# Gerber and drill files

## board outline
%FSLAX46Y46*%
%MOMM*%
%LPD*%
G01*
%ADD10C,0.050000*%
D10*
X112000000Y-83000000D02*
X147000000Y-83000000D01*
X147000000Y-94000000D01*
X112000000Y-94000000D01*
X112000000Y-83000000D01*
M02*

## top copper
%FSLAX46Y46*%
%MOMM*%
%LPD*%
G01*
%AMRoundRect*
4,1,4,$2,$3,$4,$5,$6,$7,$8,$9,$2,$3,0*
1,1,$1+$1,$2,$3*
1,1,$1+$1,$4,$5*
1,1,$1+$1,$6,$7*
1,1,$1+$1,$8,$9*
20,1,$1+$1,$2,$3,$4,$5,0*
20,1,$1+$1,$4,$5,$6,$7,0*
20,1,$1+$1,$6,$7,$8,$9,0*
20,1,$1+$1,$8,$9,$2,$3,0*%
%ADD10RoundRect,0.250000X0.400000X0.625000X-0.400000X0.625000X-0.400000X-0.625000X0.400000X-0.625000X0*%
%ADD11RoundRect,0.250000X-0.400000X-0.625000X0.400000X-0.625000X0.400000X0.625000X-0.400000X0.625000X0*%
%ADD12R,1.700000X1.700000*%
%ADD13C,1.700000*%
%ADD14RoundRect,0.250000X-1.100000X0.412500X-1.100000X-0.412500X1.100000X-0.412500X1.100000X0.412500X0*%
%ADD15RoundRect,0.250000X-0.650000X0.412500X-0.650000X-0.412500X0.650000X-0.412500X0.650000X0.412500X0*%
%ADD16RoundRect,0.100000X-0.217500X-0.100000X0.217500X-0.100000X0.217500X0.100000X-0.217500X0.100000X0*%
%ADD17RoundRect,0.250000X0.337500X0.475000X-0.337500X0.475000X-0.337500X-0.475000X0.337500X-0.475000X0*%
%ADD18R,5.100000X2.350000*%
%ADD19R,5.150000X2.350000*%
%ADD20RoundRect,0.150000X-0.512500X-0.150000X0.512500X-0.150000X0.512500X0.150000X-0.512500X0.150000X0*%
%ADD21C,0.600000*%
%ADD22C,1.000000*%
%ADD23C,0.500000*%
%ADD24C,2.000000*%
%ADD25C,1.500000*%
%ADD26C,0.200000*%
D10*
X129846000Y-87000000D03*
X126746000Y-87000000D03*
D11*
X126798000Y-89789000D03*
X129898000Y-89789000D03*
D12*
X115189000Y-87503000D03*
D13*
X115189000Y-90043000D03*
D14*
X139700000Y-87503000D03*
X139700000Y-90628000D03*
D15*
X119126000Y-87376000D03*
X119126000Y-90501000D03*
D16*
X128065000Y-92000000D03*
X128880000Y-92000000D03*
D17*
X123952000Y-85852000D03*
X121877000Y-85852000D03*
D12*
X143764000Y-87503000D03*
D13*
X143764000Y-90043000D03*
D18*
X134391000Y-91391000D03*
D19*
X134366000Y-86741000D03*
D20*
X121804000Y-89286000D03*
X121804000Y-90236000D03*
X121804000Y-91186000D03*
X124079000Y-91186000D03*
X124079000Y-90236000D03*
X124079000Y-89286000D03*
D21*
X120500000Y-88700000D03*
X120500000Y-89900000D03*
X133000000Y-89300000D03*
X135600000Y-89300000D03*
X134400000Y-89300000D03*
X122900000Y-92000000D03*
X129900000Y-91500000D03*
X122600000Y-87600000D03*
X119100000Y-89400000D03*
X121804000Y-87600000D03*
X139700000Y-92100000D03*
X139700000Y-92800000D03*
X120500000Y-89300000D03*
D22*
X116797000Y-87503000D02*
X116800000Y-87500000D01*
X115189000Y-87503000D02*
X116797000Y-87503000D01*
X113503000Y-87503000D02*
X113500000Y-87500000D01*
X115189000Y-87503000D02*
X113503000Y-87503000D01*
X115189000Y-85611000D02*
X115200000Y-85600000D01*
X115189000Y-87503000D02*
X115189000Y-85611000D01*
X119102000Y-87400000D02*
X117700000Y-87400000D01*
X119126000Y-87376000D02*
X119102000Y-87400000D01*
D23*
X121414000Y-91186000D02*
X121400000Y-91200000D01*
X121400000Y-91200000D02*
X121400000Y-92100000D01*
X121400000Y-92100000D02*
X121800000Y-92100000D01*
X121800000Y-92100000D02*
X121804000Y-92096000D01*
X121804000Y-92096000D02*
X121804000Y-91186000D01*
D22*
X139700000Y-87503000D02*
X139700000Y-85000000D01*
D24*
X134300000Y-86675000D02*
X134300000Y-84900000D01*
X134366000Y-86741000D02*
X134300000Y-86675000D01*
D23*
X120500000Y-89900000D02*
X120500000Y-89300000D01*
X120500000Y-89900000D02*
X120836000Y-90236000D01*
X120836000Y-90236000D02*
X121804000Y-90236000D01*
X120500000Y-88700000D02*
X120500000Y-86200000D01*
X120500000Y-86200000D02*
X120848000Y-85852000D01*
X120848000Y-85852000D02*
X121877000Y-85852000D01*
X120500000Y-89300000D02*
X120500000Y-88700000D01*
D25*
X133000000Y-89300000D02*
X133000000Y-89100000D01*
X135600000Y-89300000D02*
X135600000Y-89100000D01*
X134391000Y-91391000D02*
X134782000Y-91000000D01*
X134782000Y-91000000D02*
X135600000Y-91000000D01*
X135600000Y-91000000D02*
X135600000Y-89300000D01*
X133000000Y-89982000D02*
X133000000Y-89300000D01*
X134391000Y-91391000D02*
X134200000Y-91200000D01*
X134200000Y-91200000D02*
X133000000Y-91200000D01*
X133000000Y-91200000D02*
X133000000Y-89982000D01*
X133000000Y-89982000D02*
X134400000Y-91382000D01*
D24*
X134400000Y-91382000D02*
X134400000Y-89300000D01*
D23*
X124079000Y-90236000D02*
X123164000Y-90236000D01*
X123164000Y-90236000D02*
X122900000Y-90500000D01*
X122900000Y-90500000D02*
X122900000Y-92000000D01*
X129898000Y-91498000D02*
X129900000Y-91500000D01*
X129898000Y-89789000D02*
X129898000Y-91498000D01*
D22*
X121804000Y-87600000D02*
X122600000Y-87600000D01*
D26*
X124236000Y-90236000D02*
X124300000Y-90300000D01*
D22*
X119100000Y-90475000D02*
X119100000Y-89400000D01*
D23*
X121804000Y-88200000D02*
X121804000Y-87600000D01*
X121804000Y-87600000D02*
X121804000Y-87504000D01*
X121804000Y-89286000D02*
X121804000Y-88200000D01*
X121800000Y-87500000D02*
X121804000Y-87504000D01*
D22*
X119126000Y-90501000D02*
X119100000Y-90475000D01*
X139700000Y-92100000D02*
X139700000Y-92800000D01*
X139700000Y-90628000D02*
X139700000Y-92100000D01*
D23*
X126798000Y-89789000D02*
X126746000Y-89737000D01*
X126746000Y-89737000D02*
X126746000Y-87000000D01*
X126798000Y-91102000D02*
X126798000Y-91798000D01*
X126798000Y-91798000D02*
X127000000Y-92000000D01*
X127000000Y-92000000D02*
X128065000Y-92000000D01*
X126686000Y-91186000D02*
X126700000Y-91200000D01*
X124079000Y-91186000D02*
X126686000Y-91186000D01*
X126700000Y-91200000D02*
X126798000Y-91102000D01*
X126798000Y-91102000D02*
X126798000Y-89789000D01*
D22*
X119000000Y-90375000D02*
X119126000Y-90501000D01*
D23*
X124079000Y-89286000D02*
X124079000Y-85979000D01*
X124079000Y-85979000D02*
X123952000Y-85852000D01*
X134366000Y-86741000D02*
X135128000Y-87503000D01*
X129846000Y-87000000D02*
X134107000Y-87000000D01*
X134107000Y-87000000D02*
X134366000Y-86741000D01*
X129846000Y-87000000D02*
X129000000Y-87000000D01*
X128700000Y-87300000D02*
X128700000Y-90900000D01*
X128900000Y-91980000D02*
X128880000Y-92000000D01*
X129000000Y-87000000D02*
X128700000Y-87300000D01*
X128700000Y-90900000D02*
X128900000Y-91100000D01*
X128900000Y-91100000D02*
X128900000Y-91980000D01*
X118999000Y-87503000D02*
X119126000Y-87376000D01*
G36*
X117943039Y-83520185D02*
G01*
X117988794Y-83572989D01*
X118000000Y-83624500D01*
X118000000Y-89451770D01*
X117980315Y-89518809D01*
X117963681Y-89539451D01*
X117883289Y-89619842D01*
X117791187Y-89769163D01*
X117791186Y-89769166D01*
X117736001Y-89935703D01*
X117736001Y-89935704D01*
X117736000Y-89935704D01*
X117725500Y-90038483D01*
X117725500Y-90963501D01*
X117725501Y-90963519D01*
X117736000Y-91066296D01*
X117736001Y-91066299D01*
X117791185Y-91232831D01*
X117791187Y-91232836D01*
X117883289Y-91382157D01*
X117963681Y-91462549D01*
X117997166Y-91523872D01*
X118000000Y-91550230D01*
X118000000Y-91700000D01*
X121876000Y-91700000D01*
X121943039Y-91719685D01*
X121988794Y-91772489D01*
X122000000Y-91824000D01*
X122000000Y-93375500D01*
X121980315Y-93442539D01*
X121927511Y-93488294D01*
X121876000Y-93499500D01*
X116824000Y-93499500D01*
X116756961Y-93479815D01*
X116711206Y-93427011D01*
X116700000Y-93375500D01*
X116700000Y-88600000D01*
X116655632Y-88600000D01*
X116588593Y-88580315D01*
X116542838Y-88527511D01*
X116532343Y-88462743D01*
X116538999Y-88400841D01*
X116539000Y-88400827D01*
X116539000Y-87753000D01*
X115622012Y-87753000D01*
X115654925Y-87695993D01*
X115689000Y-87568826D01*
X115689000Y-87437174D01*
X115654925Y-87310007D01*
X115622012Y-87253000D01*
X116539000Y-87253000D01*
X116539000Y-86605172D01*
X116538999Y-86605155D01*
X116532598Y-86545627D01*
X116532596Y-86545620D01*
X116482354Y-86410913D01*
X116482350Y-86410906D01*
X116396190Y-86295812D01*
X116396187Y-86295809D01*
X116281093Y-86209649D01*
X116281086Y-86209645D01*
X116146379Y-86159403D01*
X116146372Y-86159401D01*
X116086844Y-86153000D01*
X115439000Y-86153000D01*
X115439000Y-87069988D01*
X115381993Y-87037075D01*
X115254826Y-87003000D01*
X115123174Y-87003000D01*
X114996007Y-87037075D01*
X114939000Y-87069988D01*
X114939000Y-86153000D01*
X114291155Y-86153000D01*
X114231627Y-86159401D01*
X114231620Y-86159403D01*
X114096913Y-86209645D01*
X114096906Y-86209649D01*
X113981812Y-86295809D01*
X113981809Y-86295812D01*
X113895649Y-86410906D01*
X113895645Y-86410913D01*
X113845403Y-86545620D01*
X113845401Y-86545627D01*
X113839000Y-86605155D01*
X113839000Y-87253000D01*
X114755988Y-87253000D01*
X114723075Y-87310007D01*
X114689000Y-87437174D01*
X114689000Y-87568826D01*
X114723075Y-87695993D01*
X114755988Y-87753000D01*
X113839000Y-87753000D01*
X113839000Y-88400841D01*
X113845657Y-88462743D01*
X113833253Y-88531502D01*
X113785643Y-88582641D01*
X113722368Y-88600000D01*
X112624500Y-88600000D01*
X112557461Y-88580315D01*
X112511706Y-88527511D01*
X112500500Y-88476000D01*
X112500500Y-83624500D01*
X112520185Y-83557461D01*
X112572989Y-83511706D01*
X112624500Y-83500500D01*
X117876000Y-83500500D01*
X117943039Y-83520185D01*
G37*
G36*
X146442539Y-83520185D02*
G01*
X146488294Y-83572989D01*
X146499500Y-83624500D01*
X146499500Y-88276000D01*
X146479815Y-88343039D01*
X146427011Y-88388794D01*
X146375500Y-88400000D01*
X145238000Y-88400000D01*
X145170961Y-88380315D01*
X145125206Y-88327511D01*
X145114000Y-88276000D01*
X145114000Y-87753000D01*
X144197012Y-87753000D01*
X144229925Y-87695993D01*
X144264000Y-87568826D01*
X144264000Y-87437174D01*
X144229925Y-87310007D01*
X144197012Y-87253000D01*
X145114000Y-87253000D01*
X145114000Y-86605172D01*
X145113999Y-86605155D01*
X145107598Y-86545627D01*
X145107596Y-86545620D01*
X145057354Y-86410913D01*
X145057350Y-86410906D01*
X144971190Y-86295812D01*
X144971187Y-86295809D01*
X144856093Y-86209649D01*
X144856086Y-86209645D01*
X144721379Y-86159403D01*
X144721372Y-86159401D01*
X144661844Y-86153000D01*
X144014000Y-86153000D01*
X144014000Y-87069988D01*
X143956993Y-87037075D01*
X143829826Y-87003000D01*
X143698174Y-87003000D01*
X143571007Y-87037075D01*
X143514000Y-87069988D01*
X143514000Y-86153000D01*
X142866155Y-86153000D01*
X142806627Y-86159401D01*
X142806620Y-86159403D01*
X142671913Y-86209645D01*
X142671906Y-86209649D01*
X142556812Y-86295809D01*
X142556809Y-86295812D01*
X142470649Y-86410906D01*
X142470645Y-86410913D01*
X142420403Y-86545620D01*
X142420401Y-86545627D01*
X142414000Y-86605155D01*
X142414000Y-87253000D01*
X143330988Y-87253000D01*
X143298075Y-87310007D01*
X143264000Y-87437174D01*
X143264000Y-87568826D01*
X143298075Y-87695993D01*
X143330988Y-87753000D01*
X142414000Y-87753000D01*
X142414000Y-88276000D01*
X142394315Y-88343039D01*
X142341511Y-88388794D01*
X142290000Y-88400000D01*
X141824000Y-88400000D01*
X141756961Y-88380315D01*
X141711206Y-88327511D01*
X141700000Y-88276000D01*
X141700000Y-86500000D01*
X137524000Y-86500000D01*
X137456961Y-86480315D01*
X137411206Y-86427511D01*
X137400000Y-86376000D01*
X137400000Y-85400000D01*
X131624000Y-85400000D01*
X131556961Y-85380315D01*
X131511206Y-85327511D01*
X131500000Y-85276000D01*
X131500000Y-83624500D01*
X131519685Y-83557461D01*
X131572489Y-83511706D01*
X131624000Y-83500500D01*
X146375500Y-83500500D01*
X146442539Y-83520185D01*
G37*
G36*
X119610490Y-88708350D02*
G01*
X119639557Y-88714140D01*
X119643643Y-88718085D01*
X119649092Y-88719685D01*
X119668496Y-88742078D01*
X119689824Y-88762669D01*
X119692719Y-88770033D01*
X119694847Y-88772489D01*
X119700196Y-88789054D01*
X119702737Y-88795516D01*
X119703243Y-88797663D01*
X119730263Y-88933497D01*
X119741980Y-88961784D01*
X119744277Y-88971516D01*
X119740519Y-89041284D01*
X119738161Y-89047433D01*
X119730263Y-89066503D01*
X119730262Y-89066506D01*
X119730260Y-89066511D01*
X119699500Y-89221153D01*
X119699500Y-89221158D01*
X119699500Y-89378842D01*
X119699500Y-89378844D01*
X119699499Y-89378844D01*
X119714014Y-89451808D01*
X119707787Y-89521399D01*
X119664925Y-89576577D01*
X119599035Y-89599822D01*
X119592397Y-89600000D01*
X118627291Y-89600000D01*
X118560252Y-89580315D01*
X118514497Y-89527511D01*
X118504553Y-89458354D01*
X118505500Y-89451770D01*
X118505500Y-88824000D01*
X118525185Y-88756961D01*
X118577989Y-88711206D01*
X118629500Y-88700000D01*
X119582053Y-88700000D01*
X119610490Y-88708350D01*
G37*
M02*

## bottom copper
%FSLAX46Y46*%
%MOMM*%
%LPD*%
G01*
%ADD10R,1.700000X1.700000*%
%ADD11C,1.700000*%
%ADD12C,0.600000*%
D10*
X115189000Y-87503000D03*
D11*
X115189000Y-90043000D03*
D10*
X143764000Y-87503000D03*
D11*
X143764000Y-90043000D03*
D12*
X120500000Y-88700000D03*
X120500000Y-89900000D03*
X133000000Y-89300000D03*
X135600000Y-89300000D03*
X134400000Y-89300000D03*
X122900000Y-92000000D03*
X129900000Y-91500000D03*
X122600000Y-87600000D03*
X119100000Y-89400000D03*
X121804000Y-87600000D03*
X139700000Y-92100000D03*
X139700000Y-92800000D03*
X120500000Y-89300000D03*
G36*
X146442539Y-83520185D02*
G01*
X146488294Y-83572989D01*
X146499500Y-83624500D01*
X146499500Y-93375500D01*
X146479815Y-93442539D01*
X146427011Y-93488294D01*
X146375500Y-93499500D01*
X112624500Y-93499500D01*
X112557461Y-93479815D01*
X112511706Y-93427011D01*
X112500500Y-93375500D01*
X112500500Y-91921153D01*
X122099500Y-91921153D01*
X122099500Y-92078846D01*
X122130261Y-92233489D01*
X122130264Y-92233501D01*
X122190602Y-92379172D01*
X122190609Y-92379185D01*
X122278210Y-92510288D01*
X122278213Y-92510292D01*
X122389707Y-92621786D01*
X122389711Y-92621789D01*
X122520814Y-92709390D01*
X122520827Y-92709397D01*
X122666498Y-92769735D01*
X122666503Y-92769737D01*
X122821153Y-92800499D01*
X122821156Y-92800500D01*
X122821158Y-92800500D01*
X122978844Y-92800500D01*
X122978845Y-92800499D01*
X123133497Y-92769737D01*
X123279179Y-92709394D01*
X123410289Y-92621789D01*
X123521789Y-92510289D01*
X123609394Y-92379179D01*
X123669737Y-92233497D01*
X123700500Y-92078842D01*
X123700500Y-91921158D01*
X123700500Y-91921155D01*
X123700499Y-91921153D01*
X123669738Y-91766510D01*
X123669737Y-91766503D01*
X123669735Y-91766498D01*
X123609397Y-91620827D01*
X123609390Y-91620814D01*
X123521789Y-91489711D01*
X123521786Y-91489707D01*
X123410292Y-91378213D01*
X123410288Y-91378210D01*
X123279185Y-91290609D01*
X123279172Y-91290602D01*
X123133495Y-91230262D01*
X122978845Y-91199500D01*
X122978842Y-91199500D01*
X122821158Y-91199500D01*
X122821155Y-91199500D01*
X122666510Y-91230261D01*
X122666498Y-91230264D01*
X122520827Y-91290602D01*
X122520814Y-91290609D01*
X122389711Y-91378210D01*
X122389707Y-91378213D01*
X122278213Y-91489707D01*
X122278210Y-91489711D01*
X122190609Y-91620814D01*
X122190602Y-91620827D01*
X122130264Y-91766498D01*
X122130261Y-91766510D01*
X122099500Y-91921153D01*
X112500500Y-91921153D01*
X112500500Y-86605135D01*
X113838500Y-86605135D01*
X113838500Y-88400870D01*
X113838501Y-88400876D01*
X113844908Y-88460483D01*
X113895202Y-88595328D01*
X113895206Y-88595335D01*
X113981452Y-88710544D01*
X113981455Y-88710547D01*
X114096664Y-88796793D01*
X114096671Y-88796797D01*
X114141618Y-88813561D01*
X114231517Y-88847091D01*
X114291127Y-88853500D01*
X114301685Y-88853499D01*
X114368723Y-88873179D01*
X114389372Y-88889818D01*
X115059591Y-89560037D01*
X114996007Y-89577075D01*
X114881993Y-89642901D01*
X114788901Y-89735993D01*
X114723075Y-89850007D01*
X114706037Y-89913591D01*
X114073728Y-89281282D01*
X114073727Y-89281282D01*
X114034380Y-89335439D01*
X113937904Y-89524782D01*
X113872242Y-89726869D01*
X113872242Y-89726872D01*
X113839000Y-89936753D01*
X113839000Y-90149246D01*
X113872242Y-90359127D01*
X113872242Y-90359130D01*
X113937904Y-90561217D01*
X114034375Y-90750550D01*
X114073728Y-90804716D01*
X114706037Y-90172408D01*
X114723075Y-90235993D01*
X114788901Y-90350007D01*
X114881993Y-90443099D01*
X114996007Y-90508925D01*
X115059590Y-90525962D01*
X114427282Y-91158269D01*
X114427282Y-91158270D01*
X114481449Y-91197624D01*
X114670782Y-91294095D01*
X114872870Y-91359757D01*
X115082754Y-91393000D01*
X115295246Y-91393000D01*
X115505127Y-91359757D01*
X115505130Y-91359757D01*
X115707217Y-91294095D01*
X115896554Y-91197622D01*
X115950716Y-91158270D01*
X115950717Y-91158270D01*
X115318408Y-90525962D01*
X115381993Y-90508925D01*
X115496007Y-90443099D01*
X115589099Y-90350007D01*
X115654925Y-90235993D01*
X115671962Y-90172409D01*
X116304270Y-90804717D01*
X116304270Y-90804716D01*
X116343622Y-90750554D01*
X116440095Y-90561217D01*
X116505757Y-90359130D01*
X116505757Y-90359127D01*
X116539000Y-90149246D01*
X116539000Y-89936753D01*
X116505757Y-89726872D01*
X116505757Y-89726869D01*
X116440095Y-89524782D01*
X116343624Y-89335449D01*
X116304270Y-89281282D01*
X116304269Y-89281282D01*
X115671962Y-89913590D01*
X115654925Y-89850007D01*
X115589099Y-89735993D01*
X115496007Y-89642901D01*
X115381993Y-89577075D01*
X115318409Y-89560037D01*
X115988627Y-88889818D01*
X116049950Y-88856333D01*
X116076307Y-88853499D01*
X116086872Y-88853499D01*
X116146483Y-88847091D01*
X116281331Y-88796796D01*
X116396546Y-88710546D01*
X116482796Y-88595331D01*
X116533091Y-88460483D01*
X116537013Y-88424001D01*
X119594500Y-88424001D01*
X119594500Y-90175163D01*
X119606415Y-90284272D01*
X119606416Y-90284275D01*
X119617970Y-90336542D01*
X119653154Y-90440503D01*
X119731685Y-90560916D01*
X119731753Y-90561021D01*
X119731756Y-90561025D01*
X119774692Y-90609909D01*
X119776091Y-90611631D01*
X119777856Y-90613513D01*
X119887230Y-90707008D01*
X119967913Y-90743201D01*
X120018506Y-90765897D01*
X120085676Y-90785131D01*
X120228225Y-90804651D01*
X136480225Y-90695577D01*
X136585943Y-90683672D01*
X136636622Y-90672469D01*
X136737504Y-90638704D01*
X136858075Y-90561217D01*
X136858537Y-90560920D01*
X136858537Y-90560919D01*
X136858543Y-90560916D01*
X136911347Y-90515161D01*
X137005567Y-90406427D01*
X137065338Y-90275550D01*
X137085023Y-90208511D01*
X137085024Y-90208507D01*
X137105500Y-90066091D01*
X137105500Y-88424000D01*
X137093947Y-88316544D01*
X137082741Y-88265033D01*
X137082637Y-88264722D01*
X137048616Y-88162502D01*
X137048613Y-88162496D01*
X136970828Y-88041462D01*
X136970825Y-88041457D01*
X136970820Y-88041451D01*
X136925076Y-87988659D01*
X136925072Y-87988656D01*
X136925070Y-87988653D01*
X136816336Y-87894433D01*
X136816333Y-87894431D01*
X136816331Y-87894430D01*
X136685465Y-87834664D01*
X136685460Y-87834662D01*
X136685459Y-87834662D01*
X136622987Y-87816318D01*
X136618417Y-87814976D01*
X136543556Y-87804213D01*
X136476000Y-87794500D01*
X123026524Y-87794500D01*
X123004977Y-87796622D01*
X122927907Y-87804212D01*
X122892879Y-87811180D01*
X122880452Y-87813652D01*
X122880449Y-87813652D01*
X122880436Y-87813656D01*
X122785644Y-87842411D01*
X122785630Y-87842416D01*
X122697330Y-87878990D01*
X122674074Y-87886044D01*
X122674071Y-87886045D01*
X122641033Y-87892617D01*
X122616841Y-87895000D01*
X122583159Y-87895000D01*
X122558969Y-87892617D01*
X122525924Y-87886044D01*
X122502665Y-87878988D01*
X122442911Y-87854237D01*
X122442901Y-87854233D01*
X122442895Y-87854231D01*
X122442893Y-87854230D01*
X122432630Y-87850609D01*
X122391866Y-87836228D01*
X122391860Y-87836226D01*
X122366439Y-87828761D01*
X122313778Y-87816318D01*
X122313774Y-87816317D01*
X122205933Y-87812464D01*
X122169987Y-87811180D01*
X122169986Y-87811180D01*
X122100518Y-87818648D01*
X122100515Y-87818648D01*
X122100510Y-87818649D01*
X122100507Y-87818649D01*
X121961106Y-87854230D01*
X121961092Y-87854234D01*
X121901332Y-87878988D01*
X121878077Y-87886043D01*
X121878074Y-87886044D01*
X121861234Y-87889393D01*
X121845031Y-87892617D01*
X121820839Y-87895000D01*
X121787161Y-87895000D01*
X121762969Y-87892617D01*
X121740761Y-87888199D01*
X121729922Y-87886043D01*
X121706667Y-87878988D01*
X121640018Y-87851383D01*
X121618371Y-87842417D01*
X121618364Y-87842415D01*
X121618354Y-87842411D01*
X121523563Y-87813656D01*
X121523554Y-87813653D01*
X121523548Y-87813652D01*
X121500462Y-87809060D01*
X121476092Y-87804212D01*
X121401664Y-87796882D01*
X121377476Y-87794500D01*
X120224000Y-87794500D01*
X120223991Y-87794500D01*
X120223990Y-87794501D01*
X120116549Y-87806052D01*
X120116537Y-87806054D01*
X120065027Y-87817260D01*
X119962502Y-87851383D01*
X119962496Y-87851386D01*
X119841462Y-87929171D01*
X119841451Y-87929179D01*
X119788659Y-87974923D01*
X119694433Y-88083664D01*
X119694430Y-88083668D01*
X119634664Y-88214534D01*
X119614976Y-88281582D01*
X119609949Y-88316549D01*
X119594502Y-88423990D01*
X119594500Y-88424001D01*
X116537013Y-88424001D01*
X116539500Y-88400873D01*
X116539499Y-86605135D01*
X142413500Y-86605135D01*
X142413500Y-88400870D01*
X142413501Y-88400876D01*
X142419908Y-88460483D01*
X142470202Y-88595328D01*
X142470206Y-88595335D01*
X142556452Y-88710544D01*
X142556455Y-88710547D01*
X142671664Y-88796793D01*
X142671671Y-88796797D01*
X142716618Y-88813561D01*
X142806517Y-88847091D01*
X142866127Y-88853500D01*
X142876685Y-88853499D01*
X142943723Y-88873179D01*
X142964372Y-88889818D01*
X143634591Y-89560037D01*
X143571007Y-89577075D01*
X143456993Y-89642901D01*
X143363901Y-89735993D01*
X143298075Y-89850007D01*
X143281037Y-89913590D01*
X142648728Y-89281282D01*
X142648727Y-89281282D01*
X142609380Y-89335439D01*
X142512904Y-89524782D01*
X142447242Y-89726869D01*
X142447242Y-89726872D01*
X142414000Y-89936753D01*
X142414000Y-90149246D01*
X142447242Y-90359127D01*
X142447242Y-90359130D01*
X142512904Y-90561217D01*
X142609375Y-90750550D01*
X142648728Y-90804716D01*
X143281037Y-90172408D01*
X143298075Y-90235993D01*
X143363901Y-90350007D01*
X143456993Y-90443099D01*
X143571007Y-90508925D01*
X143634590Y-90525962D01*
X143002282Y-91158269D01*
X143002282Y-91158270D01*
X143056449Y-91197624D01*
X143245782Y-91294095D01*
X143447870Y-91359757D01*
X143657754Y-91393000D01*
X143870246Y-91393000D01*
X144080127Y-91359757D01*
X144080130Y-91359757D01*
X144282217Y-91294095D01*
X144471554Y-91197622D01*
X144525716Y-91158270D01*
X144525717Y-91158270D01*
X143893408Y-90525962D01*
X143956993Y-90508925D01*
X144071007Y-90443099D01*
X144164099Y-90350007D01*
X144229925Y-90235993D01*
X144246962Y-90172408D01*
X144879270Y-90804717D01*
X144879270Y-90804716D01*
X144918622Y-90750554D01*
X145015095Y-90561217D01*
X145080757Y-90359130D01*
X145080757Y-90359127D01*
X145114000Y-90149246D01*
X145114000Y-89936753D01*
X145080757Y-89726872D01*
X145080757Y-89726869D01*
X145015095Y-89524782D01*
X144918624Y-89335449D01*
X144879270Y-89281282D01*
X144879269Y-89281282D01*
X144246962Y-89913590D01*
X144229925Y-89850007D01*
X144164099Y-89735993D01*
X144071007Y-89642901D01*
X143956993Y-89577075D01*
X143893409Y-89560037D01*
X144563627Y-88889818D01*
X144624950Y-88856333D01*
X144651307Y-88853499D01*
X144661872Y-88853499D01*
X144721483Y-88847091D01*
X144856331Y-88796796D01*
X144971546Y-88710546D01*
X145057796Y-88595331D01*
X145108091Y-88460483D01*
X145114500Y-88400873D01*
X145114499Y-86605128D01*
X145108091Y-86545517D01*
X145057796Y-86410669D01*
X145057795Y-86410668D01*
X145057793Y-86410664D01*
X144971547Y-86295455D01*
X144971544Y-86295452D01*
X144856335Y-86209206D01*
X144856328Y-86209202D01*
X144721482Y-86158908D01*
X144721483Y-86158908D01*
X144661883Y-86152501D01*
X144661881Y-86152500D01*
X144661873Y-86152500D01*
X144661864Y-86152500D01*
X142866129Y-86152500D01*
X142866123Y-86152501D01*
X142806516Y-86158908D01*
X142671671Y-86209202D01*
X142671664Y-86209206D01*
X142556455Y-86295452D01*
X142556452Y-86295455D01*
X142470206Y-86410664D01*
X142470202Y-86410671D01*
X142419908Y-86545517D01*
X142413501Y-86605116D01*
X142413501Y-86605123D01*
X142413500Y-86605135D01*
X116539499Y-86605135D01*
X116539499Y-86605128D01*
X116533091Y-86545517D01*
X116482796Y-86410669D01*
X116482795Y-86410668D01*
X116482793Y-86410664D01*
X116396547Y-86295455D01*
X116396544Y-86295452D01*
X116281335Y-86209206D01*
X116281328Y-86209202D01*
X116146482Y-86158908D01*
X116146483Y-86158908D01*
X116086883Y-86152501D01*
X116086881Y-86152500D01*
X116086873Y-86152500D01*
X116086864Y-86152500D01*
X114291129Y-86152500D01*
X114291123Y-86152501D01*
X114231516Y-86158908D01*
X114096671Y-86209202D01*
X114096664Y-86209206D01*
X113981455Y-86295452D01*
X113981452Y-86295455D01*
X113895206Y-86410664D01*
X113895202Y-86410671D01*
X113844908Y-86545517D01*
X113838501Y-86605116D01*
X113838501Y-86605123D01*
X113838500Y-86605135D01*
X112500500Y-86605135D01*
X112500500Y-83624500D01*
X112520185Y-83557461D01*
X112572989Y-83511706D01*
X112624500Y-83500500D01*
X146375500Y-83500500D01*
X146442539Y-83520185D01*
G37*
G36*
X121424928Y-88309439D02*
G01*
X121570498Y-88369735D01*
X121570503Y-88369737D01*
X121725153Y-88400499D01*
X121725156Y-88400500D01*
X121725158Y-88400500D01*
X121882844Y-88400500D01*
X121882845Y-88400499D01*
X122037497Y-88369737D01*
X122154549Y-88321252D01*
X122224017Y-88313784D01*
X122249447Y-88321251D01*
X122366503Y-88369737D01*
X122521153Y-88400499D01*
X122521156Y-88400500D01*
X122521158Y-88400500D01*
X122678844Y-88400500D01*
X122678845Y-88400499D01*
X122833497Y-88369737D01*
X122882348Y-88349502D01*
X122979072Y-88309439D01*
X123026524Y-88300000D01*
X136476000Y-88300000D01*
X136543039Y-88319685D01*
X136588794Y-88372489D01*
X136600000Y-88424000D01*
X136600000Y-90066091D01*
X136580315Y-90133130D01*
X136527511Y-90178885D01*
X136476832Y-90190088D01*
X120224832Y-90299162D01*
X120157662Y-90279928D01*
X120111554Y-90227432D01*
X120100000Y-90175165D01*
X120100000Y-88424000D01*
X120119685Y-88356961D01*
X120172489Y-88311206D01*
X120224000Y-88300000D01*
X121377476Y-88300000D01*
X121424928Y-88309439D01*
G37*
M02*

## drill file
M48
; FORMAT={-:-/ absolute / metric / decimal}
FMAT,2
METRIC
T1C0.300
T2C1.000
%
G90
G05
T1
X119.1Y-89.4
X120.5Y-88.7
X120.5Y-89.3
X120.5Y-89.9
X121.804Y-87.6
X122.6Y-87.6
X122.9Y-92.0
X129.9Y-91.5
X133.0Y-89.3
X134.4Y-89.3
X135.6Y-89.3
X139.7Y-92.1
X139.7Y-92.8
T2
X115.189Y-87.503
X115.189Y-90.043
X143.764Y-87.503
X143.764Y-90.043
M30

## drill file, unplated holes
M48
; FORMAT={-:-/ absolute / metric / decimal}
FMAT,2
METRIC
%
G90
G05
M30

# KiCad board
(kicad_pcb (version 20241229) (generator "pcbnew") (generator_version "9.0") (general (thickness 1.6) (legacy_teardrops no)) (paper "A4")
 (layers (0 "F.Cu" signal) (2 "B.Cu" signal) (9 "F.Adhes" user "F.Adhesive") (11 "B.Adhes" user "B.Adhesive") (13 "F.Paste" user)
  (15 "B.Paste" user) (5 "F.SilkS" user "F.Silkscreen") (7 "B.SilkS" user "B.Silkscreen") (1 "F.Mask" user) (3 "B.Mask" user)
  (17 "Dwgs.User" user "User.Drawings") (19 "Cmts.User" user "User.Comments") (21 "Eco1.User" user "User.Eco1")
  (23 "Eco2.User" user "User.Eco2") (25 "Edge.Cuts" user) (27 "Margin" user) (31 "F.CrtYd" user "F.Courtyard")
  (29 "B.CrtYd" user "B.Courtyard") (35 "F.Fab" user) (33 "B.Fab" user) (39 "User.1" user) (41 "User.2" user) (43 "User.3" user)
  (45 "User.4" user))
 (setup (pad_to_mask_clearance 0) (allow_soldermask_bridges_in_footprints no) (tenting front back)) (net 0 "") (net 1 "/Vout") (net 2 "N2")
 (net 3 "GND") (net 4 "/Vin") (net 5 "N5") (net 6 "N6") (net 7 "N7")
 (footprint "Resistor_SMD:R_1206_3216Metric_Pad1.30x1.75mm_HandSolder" (layer "F.Cu") (at 128.296 87 180)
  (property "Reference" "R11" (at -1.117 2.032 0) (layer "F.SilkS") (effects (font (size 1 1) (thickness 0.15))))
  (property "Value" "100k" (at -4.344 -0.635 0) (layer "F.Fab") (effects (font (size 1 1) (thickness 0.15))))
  (pad "1" smd roundrect (at -1.55 0 180) (size 1.3 1.75) (layers "F.Cu" "F.Mask" "F.Paste") (roundrect_rratio 0.192308) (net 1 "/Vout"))
  (pad "2" smd roundrect (at 1.55 0 180) (size 1.3 1.75) (layers "F.Cu" "F.Mask" "F.Paste") (roundrect_rratio 0.192308) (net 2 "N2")))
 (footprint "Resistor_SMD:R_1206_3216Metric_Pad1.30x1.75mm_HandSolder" (layer "F.Cu") (at 128.348 89.789)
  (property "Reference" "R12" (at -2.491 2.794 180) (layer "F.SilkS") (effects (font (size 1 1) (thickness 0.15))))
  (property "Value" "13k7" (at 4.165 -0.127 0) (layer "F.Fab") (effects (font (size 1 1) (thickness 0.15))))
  (pad "1" smd roundrect (at -1.55 0) (size 1.3 1.75) (layers "F.Cu" "F.Mask" "F.Paste") (roundrect_rratio 0.192308) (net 2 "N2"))
  (pad "2" smd roundrect (at 1.55 0) (size 1.3 1.75) (layers "F.Cu" "F.Mask" "F.Paste") (roundrect_rratio 0.192308) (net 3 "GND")))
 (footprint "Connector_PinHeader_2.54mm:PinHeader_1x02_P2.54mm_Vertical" (layer "F.Cu") (at 115.189 87.503)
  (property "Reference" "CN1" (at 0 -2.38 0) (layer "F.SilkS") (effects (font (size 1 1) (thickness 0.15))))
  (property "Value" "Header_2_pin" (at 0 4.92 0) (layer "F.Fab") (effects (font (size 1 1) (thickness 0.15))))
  (pad "1" thru_hole rect (at 0 0) (size 1.7 1.7) (drill 1) (layers "*.Cu" "*.Mask") (remove_unused_layers no) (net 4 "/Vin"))
  (pad "2" thru_hole circle (at 0 2.54) (size 1.7 1.7) (drill 1) (layers "*.Cu" "*.Mask") (remove_unused_layers no) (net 3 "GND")))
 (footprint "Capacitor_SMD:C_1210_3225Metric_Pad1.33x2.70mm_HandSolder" (layer "F.Cu") (at 139.7 89.0655 -90)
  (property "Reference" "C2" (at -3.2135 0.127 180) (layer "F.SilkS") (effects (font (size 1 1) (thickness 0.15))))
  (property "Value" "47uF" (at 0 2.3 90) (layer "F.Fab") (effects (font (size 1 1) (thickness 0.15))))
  (pad "1" smd roundrect (at -1.5625 0 270) (size 1.325 2.7) (layers "F.Cu" "F.Mask" "F.Paste") (roundrect_rratio 0.188679) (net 1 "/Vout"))
  (pad "2" smd roundrect (at 1.5625 0 270) (size 1.325 2.7) (layers "F.Cu" "F.Mask" "F.Paste") (roundrect_rratio 0.188679) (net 3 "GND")))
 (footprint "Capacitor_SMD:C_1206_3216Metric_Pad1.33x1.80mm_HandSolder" (layer "F.Cu") (at 119.126 88.9385 -90)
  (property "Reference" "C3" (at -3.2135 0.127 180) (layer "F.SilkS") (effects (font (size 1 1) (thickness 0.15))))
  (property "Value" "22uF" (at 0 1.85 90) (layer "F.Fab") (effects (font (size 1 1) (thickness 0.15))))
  (pad "1" smd roundrect (at -1.5625 0 270) (size 1.325 1.8) (layers "F.Cu" "F.Mask" "F.Paste") (roundrect_rratio 0.188679) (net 4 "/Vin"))
  (pad "2" smd roundrect (at 1.5625 0 270) (size 1.325 1.8) (layers "F.Cu" "F.Mask" "F.Paste") (roundrect_rratio 0.188679) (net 3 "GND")))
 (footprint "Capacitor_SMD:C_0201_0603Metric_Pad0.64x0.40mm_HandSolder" (layer "F.Cu") (at 128.4725 92)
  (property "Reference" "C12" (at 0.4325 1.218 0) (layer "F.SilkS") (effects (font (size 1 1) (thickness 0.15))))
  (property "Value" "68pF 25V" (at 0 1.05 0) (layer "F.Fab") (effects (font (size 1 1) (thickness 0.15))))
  (pad "" smd roundrect (at -0.4325 0) (size 0.458 0.36) (layers "F.Paste") (roundrect_rratio 0.25))
  (pad "" smd roundrect (at 0.4325 0) (size 0.458 0.36) (layers "F.Paste") (roundrect_rratio 0.25))
  (pad "1" smd roundrect (at -0.4075 0) (size 0.635 0.4) (layers "F.Cu" "F.Mask") (roundrect_rratio 0.25) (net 2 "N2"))
  (pad "2" smd roundrect (at 0.4075 0) (size 0.635 0.4) (layers "F.Cu" "F.Mask") (roundrect_rratio 0.25) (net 1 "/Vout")))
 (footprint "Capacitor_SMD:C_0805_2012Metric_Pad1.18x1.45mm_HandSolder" (layer "F.Cu") (at 122.9145 85.852 180)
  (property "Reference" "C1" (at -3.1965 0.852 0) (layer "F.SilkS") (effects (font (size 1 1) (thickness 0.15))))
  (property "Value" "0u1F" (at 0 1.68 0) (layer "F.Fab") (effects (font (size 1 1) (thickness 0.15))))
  (pad "1" smd roundrect (at -1.0375 0 180) (size 1.175 1.45) (layers "F.Cu" "F.Mask" "F.Paste") (roundrect_rratio 0.212766) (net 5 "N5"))
  (pad "2" smd roundrect (at 1.0375 0 180) (size 1.175 1.45) (layers "F.Cu" "F.Mask" "F.Paste") (roundrect_rratio 0.212766) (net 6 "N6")))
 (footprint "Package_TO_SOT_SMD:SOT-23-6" (layer "F.Cu") (at 122.9415 90.236)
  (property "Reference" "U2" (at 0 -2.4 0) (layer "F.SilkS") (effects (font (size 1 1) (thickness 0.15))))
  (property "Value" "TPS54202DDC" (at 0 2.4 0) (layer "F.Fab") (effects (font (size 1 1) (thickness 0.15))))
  (pad "1" smd roundrect (at -1.1375 -0.95) (size 1.325 0.6) (layers "F.Cu" "F.Mask" "F.Paste") (roundrect_rratio 0.25) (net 3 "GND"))
  (pad "2" smd roundrect (at -1.1375 0) (size 1.325 0.6) (layers "F.Cu" "F.Mask" "F.Paste") (roundrect_rratio 0.25) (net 6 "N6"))
  (pad "3" smd roundrect (at -1.1375 0.95) (size 1.325 0.6) (layers "F.Cu" "F.Mask" "F.Paste") (roundrect_rratio 0.25) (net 4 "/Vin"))
  (pad "4" smd roundrect (at 1.1375 0.95) (size 1.325 0.6) (layers "F.Cu" "F.Mask" "F.Paste") (roundrect_rratio 0.25) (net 2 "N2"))
  (pad "5" smd roundrect (at 1.1375 0) (size 1.325 0.6) (layers "F.Cu" "F.Mask" "F.Paste") (roundrect_rratio 0.25) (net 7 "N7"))
  (pad "6" smd roundrect (at 1.1375 -0.95) (size 1.325 0.6) (layers "F.Cu" "F.Mask" "F.Paste") (roundrect_rratio 0.25) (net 5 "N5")))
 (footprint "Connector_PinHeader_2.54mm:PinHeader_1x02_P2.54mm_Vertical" (layer "F.Cu") (at 143.764 87.503)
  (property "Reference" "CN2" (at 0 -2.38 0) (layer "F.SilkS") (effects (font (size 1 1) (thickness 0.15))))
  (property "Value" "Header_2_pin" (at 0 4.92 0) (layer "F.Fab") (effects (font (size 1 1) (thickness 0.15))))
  (pad "1" thru_hole rect (at 0 0) (size 1.7 1.7) (drill 1) (layers "*.Cu" "*.Mask") (remove_unused_layers no) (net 1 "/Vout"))
  (pad "2" thru_hole circle (at 0 2.54) (size 1.7 1.7) (drill 1) (layers "*.Cu" "*.Mask") (remove_unused_layers no) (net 3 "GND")))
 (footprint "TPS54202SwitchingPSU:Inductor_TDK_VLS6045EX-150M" (layer "F.Cu") (at 134.391 89.066 90)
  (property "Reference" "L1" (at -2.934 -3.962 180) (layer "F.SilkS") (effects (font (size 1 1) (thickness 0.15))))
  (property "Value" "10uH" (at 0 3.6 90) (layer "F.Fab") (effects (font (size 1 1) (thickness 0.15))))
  (pad "1" smd rect (at -2.325 0 90) (size 2.35 5.1) (layers "F.Cu" "F.Mask" "F.Paste") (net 6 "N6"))
  (pad "2" smd rect (at 2.325 -0.025 90) (size 2.35 5.15) (layers "F.Cu" "F.Mask" "F.Paste") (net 1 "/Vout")))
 (gr_rect (start 112 83) (end 147 94) (stroke (width 0.05) (type default)) (fill no) (layer "Edge.Cuts"))
 (segment (start 120.5 89.9) (end 120.5 89.3) (width 0.5) (layer "F.Cu") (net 6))
 (segment (start 133 89.3) (end 133 89.1) (width 1.5) (layer "F.Cu") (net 6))
 (segment (start 133 89.982) (end 134.4 91.382) (width 1.5) (layer "F.Cu") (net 6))
 (segment (start 120.5 89.9) (end 120.836 90.236) (width 0.5) (layer "F.Cu") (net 6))
 (segment (start 134.391 91.391) (end 134.2 91.2) (width 1.5) (layer "F.Cu") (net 6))
 (segment (start 120.5 86.2) (end 120.848 85.852) (width 0.5) (layer "F.Cu") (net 6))
 (segment (start 120.5 88.7) (end 120.5 86.2) (width 0.5) (layer "F.Cu") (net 6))
 (segment (start 120.836 90.236) (end 121.804 90.236) (width 0.5) (layer "F.Cu") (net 6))
 (segment (start 134.4 91.382) (end 134.4 89.3) (width 2) (layer "F.Cu") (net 6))
 (segment (start 133 89.982) (end 133 89.3) (width 1.5) (layer "F.Cu") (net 6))
 (segment (start 120.848 85.852) (end 121.877 85.852) (width 0.5) (layer "F.Cu") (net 6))
 (segment (start 120.5 89.3) (end 120.5 88.7) (width 0.5) (layer "F.Cu") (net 6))
 (segment (start 135.6 91) (end 135.6 89.3) (width 1.5) (layer "F.Cu") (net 6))
 (segment (start 134.391 91.391) (end 134.782 91) (width 1.5) (layer "F.Cu") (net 6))
 (segment (start 135.6 89.3) (end 135.6 89.1) (width 1.5) (layer "F.Cu") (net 6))
 (segment (start 133 91.2) (end 133 89.982) (width 1.5) (layer "F.Cu") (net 6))
 (segment (start 134.2 91.2) (end 133 91.2) (width 1.5) (layer "F.Cu") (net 6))
 (segment (start 134.782 91) (end 135.6 91) (width 1.5) (layer "F.Cu") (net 6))
 (via (at 120.5 89.9) (size 0.6) (drill 0.3) (layers "F.Cu" "B.Cu") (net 6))
 (via (at 120.5 89.3) (size 0.6) (drill 0.3) (layers "F.Cu" "B.Cu") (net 6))
 (via (at 133 89.3) (size 0.6) (drill 0.3) (layers "F.Cu" "B.Cu") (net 6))
 (via (at 135.6 89.3) (size 0.6) (drill 0.3) (layers "F.Cu" "B.Cu") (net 6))
 (via (at 134.4 89.3) (size 0.6) (drill 0.3) (layers "F.Cu" "B.Cu") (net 6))
 (via (at 120.5 88.7) (size 0.6) (drill 0.3) (layers "F.Cu" "B.Cu") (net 6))
 (segment (start 124.079 89.286) (end 124.079 85.979) (width 0.5) (layer "F.Cu") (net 5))
 (segment (start 124.079 85.979) (end 123.952 85.852) (width 0.5) (layer "F.Cu") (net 5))
 (segment (start 134.366 86.741) (end 134.3 86.675) (width 2) (layer "F.Cu") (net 1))
 (segment (start 134.107 87) (end 134.366 86.741) (width 0.5) (layer "F.Cu") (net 1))
 (segment (start 128.9 91.98) (end 128.88 92) (width 0.5) (layer "F.Cu") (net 1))
 (segment (start 139.7 87.503) (end 139.7 85) (width 1) (layer "F.Cu") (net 1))
 (segment (start 134.366 86.741) (end 135.128 87.503) (width 0.5) (layer "F.Cu") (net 1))
 (segment (start 129.846 87) (end 134.107 87) (width 0.5) (layer "F.Cu") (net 1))
 (segment (start 129 87) (end 128.7 87.3) (width 0.5) (layer "F.Cu") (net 1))
 (segment (start 129.846 87) (end 129 87) (width 0.5) (layer "F.Cu") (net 1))
 (segment (start 128.7 90.9) (end 128.9 91.1) (width 0.5) (layer "F.Cu") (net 1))
 (segment (start 128.9 91.1) (end 128.9 91.98) (width 0.5) (layer "F.Cu") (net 1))
 (segment (start 128.7 87.3) (end 128.7 90.9) (width 0.5) (layer "F.Cu") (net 1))
 (segment (start 134.3 86.675) (end 134.3 84.9) (width 2) (layer "F.Cu") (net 1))
 (segment (start 139.7 90.628) (end 139.7 92.1) (width 1) (layer "F.Cu") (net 3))
 (segment (start 129.898 89.789) (end 129.898 91.498) (width 0.5) (layer "F.Cu") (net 3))
 (segment (start 121.804 87.6) (end 121.804 87.504) (width 0.5) (layer "F.Cu") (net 3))
 (segment (start 119.1 90.475) (end 119.1 89.4) (width 1) (layer "F.Cu") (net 3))
 (segment (start 121.804 87.6) (end 122.6 87.6) (width 1) (layer "F.Cu") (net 3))
 (segment (start 121.804 89.286) (end 121.804 88.2) (width 0.5) (layer "F.Cu") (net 3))
 (segment (start 119.126 90.501) (end 119.1 90.475) (width 1) (layer "F.Cu") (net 3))
 (segment (start 121.8 87.5) (end 121.804 87.504) (width 0.5) (layer "F.Cu") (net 3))
 (segment (start 121.804 88.2) (end 121.804 87.6) (width 0.5) (layer "F.Cu") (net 3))
 (segment (start 129.898 91.498) (end 129.9 91.5) (width 0.5) (layer "F.Cu") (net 3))
 (segment (start 119 90.375) (end 119.126 90.501) (width 1) (layer "F.Cu") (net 3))
 (segment (start 139.7 92.1) (end 139.7 92.8) (width 1) (layer "F.Cu") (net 3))
 (via (at 139.7 92.1) (size 0.6) (drill 0.3) (layers "F.Cu" "B.Cu") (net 3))
 (via (at 121.804 87.6) (size 0.6) (drill 0.3) (layers "F.Cu" "B.Cu") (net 3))
 (via (at 139.7 92.8) (size 0.6) (drill 0.3) (layers "F.Cu" "B.Cu") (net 3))
 (via (at 119.1 89.4) (size 0.6) (drill 0.3) (layers "F.Cu" "B.Cu") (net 3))
 (via (at 129.9 91.5) (size 0.6) (drill 0.3) (layers "F.Cu" "B.Cu") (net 3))
 (via (at 122.6 87.6) (size 0.6) (drill 0.3) (layers "F.Cu" "B.Cu") (free yes) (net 3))
 (segment (start 121.4 91.2) (end 121.4 92.1) (width 0.5) (layer "F.Cu") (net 4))
 (segment (start 121.804 92.096) (end 121.804 91.186) (width 0.5) (layer "F.Cu") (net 4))
 (segment (start 113.503 87.503) (end 113.5 87.5) (width 1) (layer "F.Cu") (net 4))
 (segment (start 121.8 92.1) (end 121.804 92.096) (width 0.5) (layer "F.Cu") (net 4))
 (segment (start 119.102 87.4) (end 117.7 87.4) (width 1) (layer "F.Cu") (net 4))
 (segment (start 115.189 87.503) (end 116.797 87.503) (width 1) (layer "F.Cu") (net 4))
 (segment (start 115.189 87.503) (end 115.189 85.611) (width 1) (layer "F.Cu") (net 4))
 (segment (start 121.414 91.186) (end 121.4 91.2) (width 0.5) (layer "F.Cu") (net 4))
 (segment (start 116.797 87.503) (end 116.8 87.5) (width 1) (layer "F.Cu") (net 4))
 (segment (start 115.189 85.611) (end 115.2 85.6) (width 1) (layer "F.Cu") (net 4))
 (segment (start 121.4 92.1) (end 121.8 92.1) (width 0.5) (layer "F.Cu") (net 4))
 (segment (start 119.126 87.376) (end 119.102 87.4) (width 1) (layer "F.Cu") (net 4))
 (segment (start 118.999 87.503) (end 119.126 87.376) (width 0.5) (layer "F.Cu") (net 4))
 (segment (start 115.189 87.503) (end 113.503 87.503) (width 1) (layer "F.Cu") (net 4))
 (segment (start 126.798 91.102) (end 126.798 91.798) (width 0.5) (layer "F.Cu") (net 2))
 (segment (start 124.079 91.186) (end 126.686 91.186) (width 0.5) (layer "F.Cu") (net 2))
 (segment (start 126.798 91.798) (end 127 92) (width 0.5) (layer "F.Cu") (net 2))
 (segment (start 127 92) (end 128.065 92) (width 0.5) (layer "F.Cu") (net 2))
 (segment (start 126.798 89.789) (end 126.746 89.737) (width 0.5) (layer "F.Cu") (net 2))
 (segment (start 126.686 91.186) (end 126.7 91.2) (width 0.5) (layer "F.Cu") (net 2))
 (segment (start 126.746 89.737) (end 126.746 87) (width 0.5) (layer "F.Cu") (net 2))
 (segment (start 126.798 91.102) (end 126.798 89.789) (width 0.5) (layer "F.Cu") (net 2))
 (segment (start 126.7 91.2) (end 126.798 91.102) (width 0.5) (layer "F.Cu") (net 2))
 (segment (start 124.079 90.236) (end 123.164 90.236) (width 0.5) (layer "F.Cu") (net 7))
 (segment (start 122.9 90.5) (end 122.9 92) (width 0.5) (layer "F.Cu") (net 7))
 (segment (start 124.236 90.236) (end 124.3 90.3) (width 0.2) (layer "F.Cu") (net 7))
 (segment (start 123.164 90.236) (end 122.9 90.5) (width 0.5) (layer "F.Cu") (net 7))
 (via (at 122.9 92) (size 0.6) (drill 0.3) (layers "F.Cu" "B.Cu") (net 7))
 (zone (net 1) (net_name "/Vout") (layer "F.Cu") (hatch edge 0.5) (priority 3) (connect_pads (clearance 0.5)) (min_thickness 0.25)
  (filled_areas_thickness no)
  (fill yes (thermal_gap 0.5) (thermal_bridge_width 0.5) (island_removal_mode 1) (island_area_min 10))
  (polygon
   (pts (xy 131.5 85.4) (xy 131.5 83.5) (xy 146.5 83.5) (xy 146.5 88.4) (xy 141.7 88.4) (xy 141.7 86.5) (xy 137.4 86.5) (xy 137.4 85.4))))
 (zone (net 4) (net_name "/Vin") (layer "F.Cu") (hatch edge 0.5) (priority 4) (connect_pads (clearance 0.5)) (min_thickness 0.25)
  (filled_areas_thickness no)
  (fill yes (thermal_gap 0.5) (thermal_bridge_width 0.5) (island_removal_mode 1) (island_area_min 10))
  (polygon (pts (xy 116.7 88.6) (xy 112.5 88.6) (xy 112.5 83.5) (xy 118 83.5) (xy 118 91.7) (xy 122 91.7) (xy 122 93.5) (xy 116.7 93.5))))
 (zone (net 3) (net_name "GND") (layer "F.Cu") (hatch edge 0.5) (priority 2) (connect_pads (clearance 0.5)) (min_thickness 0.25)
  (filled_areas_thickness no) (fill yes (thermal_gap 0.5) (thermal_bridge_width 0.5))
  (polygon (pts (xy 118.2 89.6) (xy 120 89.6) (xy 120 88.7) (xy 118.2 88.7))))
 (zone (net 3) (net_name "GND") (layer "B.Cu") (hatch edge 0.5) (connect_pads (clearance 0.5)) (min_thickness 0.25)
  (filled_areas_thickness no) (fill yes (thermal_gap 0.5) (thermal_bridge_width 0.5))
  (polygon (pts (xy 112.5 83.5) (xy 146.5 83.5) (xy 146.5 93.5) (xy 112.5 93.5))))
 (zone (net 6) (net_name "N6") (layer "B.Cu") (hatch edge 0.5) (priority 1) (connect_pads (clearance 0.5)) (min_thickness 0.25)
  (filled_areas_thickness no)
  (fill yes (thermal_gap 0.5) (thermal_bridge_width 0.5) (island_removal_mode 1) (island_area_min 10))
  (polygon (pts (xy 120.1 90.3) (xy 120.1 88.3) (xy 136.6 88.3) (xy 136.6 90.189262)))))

